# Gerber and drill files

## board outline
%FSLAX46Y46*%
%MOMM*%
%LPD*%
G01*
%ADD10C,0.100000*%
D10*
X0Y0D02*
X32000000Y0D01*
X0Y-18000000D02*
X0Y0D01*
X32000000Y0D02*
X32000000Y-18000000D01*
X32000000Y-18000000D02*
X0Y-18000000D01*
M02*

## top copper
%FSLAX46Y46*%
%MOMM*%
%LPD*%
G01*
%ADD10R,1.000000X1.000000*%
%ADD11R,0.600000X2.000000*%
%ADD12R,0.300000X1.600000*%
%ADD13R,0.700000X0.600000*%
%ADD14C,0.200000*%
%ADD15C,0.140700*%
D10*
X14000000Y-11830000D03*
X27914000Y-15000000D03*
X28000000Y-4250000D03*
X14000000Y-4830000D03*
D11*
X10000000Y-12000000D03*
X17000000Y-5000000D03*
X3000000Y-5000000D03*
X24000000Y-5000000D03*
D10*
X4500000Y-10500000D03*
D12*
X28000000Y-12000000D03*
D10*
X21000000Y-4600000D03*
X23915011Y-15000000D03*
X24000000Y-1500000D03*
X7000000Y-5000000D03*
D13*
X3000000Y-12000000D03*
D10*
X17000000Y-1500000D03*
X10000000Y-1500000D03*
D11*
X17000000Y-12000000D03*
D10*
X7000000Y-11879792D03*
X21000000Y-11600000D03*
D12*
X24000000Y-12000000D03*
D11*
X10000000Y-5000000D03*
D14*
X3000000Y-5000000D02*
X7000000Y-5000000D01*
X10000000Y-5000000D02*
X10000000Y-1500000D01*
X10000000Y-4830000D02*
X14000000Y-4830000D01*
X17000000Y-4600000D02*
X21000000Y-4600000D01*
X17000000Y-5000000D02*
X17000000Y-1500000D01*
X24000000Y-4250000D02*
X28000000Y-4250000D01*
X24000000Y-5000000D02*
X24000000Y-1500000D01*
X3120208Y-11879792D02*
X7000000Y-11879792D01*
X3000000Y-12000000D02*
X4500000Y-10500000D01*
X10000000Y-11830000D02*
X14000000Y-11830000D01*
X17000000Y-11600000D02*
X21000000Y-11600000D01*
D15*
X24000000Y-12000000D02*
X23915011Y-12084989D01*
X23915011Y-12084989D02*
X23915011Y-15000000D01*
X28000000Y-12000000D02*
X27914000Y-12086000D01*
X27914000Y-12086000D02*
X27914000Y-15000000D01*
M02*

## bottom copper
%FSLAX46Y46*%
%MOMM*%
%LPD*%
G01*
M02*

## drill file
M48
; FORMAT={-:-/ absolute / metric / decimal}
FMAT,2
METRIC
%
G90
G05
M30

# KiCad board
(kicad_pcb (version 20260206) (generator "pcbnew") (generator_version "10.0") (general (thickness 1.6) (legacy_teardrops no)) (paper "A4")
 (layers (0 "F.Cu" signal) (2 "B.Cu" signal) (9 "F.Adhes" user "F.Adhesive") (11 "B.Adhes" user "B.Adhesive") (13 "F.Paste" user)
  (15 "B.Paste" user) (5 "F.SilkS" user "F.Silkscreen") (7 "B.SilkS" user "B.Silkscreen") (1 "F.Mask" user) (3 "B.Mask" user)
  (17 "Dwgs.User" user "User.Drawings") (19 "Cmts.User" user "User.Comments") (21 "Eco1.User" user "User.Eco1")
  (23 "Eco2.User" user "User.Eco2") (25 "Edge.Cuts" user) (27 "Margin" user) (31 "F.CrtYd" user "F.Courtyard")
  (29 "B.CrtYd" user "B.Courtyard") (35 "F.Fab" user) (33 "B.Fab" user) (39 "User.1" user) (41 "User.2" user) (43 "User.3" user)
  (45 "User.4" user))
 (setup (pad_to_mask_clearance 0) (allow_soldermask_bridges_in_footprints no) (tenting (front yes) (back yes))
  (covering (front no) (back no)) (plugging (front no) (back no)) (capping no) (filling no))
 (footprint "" (layer "F.Cu") (at 14 11.83)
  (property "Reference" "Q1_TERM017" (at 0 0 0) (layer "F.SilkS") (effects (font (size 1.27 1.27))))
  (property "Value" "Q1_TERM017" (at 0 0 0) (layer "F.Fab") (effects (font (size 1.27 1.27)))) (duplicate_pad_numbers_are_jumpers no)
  (pad "1" smd rect (at 0 0) (size 1 1) (layers "F.Cu" "F.Mask" "F.Paste") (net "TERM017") (thermal_bridge_angle 45)))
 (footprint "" (layer "F.Cu") (at 27.914 15)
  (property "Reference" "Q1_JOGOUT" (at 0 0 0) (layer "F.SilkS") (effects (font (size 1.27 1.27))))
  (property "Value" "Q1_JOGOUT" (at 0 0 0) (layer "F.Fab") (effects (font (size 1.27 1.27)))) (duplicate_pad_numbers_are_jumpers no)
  (pad "1" smd rect (at 0 0) (size 1 1) (layers "F.Cu" "F.Mask" "F.Paste") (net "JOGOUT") (thermal_bridge_angle 45)))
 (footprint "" (layer "F.Cu") (at 28 4.25)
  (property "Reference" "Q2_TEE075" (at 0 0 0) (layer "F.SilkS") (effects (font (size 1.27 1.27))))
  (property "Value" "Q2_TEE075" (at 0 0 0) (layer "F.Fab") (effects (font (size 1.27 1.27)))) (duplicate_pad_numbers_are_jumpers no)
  (pad "1" smd rect (at 0 0) (size 1 1) (layers "F.Cu" "F.Mask" "F.Paste") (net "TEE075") (thermal_bridge_angle 45)))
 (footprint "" (layer "F.Cu") (at 14 4.83)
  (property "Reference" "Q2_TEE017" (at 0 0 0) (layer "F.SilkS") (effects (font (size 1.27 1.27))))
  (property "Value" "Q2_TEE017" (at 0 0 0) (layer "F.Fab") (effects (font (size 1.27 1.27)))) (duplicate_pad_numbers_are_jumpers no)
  (pad "1" smd rect (at 0 0) (size 1 1) (layers "F.Cu" "F.Mask" "F.Paste") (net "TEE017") (thermal_bridge_angle 45)))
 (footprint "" (layer "F.Cu") (at 10 12)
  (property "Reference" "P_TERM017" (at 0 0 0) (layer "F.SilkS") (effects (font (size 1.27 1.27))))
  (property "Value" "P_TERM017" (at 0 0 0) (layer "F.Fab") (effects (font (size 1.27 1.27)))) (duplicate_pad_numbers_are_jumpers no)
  (pad "1" smd rect (at 0 0) (size 0.6 2) (layers "F.Cu" "F.Mask" "F.Paste") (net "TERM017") (thermal_bridge_angle 45)))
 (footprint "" (layer "F.Cu") (at 17 5)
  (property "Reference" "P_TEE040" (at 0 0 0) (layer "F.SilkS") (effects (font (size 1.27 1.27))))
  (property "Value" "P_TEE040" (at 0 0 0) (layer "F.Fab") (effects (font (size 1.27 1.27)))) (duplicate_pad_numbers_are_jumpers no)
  (pad "1" smd rect (at 0 0) (size 0.6 2) (layers "F.Cu" "F.Mask" "F.Paste") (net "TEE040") (thermal_bridge_angle 45)))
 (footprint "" (layer "F.Cu") (at 3 5)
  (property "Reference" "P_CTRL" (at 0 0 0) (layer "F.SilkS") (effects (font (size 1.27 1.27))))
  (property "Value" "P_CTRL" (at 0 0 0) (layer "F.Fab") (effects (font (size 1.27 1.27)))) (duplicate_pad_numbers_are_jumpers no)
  (pad "1" smd rect (at 0 0) (size 0.6 2) (layers "F.Cu" "F.Mask" "F.Paste") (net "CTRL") (thermal_bridge_angle 45)))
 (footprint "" (layer "F.Cu") (at 24 5)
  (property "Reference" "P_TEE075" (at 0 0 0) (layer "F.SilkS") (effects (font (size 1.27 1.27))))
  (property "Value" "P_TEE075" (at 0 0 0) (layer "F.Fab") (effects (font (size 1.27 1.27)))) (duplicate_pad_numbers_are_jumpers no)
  (pad "1" smd rect (at 0 0) (size 0.6 2) (layers "F.Cu" "F.Mask" "F.Paste") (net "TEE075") (thermal_bridge_angle 45)))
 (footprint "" (layer "F.Cu") (at 4.5 10.5)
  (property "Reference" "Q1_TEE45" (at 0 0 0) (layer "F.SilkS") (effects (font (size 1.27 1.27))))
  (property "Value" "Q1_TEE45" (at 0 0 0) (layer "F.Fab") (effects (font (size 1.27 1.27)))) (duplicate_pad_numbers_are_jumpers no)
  (pad "1" smd rect (at 0 0) (size 1 1) (layers "F.Cu" "F.Mask" "F.Paste") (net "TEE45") (thermal_bridge_angle 45)))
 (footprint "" (layer "F.Cu") (at 28 12)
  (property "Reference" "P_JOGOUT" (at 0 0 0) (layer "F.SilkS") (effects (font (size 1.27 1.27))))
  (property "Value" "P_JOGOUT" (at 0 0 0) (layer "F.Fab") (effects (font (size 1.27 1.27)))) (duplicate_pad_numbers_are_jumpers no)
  (pad "1" smd rect (at 0 0) (size 0.3 1.6) (layers "F.Cu" "F.Mask" "F.Paste") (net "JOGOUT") (thermal_bridge_angle 45)))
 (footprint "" (layer "F.Cu") (at 21 4.6)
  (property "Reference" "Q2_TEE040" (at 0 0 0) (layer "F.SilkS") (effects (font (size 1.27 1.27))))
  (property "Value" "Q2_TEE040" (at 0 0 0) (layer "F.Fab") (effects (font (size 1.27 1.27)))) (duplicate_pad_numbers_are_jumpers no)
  (pad "1" smd rect (at 0 0) (size 1 1) (layers "F.Cu" "F.Mask" "F.Paste") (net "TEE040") (thermal_bridge_angle 45)))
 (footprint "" (layer "F.Cu") (at 23.915011 15)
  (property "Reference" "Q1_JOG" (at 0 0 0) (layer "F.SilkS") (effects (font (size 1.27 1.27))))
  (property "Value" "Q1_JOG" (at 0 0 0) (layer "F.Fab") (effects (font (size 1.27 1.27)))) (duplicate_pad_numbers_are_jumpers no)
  (pad "1" smd rect (at 0 0) (size 1 1) (layers "F.Cu" "F.Mask" "F.Paste") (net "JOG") (thermal_bridge_angle 45)))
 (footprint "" (layer "F.Cu") (at 24 1.5)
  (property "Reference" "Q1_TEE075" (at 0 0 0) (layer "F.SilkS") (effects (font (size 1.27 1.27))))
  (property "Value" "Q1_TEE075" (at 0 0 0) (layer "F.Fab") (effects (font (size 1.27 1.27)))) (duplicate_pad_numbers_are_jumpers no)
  (pad "1" smd rect (at 0 0) (size 1 1) (layers "F.Cu" "F.Mask" "F.Paste") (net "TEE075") (thermal_bridge_angle 45)))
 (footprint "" (layer "F.Cu") (at 7 5)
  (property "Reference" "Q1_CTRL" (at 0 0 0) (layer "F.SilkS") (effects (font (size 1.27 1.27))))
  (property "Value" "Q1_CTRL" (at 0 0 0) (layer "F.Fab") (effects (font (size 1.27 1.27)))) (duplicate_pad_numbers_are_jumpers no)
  (pad "1" smd rect (at 0 0) (size 1 1) (layers "F.Cu" "F.Mask" "F.Paste") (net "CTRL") (thermal_bridge_angle 45)))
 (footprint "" (layer "F.Cu") (at 3 12)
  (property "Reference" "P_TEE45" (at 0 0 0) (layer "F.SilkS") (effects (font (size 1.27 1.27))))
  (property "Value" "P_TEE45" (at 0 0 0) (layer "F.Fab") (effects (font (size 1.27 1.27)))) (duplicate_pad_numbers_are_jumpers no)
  (pad "1" smd rect (at 0 0) (size 0.7 0.6) (layers "F.Cu" "F.Mask" "F.Paste") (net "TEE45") (thermal_bridge_angle 45)))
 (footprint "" (layer "F.Cu") (at 17 1.5)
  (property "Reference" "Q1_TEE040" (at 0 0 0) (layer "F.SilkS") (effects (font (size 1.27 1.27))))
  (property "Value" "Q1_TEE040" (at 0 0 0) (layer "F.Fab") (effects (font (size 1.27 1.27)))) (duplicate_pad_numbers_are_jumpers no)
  (pad "1" smd rect (at 0 0) (size 1 1) (layers "F.Cu" "F.Mask" "F.Paste") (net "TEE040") (thermal_bridge_angle 45)))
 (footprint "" (layer "F.Cu") (at 10 1.5)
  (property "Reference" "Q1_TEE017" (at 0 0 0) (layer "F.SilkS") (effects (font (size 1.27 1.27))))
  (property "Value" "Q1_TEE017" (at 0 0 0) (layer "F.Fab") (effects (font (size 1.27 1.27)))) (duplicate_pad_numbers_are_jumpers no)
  (pad "1" smd rect (at 0 0) (size 1 1) (layers "F.Cu" "F.Mask" "F.Paste") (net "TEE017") (thermal_bridge_angle 45)))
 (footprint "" (layer "F.Cu") (at 17 12)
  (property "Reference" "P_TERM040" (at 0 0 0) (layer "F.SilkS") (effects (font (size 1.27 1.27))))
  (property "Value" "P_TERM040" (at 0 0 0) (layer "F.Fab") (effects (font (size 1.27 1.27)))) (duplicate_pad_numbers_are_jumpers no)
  (pad "1" smd rect (at 0 0) (size 0.6 2) (layers "F.Cu" "F.Mask" "F.Paste") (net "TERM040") (thermal_bridge_angle 45)))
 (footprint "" (layer "F.Cu") (at 7 11.879792)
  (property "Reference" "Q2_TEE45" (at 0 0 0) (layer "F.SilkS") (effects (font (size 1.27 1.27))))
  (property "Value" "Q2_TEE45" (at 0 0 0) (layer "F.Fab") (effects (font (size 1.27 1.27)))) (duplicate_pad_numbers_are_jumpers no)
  (pad "1" smd rect (at 0 0) (size 1 1) (layers "F.Cu" "F.Mask" "F.Paste") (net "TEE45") (thermal_bridge_angle 45)))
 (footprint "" (layer "F.Cu") (at 21 11.6)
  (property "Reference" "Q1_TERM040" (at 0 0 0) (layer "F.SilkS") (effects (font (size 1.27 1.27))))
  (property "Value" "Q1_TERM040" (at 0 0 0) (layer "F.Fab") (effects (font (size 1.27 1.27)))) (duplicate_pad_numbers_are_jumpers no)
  (pad "1" smd rect (at 0 0) (size 1 1) (layers "F.Cu" "F.Mask" "F.Paste") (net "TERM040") (thermal_bridge_angle 45)))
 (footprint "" (layer "F.Cu") (at 24 12)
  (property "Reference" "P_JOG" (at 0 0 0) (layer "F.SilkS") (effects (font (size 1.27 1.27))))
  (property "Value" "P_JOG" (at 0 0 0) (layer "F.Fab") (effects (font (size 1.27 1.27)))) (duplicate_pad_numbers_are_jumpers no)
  (pad "1" smd rect (at 0 0) (size 0.3 1.6) (layers "F.Cu" "F.Mask" "F.Paste") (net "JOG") (thermal_bridge_angle 45)))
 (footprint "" (layer "F.Cu") (at 10 5)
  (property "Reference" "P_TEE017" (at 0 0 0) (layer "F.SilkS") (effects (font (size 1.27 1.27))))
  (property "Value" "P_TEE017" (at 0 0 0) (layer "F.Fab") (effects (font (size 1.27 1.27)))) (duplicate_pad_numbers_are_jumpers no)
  (pad "1" smd rect (at 0 0) (size 0.6 2) (layers "F.Cu" "F.Mask" "F.Paste") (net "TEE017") (thermal_bridge_angle 45)))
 (gr_line (start 0 0) (end 32 0) (stroke (width 0.1) (type default)) (layer "Edge.Cuts"))
 (gr_line (start 0 18) (end 0 0) (stroke (width 0.1) (type default)) (layer "Edge.Cuts"))
 (gr_line (start 32 0) (end 32 18) (stroke (width 0.1) (type default)) (layer "Edge.Cuts"))
 (gr_line (start 32 18) (end 0 18) (stroke (width 0.1) (type default)) (layer "Edge.Cuts"))
 (segment (start 3 5) (end 7 5) (width 0.2) (layer "F.Cu") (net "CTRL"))
 (segment (start 10 5) (end 10 1.5) (width 0.2) (layer "F.Cu") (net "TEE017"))
 (segment (start 10 4.83) (end 14 4.83) (width 0.2) (layer "F.Cu") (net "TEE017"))
 (segment (start 17 4.6) (end 21 4.6) (width 0.2) (layer "F.Cu") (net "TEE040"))
 (segment (start 17 5) (end 17 1.5) (width 0.2) (layer "F.Cu") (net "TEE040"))
 (segment (start 24 4.25) (end 28 4.25) (width 0.2) (layer "F.Cu") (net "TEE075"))
 (segment (start 24 5) (end 24 1.5) (width 0.2) (layer "F.Cu") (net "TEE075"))
 (segment (start 3.120208 11.879792) (end 7 11.879792) (width 0.2) (layer "F.Cu") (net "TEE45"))
 (segment (start 3 12) (end 4.5 10.5) (width 0.2) (layer "F.Cu") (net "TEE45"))
 (segment (start 10 11.83) (end 14 11.83) (width 0.2) (layer "F.Cu") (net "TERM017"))
 (segment (start 17 11.6) (end 21 11.6) (width 0.2) (layer "F.Cu") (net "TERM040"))
 (segment (start 24 12) (end 23.915011 12.084989) (width 0.1407) (layer "F.Cu") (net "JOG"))
 (segment (start 23.915011 12.084989) (end 23.915011 15) (width 0.1407) (layer "F.Cu") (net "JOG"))
 (segment (start 28 12) (end 27.914 12.086) (width 0.1407) (layer "F.Cu") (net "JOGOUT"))
 (segment (start 27.914 12.086) (end 27.914 15) (width 0.1407) (layer "F.Cu") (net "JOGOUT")))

